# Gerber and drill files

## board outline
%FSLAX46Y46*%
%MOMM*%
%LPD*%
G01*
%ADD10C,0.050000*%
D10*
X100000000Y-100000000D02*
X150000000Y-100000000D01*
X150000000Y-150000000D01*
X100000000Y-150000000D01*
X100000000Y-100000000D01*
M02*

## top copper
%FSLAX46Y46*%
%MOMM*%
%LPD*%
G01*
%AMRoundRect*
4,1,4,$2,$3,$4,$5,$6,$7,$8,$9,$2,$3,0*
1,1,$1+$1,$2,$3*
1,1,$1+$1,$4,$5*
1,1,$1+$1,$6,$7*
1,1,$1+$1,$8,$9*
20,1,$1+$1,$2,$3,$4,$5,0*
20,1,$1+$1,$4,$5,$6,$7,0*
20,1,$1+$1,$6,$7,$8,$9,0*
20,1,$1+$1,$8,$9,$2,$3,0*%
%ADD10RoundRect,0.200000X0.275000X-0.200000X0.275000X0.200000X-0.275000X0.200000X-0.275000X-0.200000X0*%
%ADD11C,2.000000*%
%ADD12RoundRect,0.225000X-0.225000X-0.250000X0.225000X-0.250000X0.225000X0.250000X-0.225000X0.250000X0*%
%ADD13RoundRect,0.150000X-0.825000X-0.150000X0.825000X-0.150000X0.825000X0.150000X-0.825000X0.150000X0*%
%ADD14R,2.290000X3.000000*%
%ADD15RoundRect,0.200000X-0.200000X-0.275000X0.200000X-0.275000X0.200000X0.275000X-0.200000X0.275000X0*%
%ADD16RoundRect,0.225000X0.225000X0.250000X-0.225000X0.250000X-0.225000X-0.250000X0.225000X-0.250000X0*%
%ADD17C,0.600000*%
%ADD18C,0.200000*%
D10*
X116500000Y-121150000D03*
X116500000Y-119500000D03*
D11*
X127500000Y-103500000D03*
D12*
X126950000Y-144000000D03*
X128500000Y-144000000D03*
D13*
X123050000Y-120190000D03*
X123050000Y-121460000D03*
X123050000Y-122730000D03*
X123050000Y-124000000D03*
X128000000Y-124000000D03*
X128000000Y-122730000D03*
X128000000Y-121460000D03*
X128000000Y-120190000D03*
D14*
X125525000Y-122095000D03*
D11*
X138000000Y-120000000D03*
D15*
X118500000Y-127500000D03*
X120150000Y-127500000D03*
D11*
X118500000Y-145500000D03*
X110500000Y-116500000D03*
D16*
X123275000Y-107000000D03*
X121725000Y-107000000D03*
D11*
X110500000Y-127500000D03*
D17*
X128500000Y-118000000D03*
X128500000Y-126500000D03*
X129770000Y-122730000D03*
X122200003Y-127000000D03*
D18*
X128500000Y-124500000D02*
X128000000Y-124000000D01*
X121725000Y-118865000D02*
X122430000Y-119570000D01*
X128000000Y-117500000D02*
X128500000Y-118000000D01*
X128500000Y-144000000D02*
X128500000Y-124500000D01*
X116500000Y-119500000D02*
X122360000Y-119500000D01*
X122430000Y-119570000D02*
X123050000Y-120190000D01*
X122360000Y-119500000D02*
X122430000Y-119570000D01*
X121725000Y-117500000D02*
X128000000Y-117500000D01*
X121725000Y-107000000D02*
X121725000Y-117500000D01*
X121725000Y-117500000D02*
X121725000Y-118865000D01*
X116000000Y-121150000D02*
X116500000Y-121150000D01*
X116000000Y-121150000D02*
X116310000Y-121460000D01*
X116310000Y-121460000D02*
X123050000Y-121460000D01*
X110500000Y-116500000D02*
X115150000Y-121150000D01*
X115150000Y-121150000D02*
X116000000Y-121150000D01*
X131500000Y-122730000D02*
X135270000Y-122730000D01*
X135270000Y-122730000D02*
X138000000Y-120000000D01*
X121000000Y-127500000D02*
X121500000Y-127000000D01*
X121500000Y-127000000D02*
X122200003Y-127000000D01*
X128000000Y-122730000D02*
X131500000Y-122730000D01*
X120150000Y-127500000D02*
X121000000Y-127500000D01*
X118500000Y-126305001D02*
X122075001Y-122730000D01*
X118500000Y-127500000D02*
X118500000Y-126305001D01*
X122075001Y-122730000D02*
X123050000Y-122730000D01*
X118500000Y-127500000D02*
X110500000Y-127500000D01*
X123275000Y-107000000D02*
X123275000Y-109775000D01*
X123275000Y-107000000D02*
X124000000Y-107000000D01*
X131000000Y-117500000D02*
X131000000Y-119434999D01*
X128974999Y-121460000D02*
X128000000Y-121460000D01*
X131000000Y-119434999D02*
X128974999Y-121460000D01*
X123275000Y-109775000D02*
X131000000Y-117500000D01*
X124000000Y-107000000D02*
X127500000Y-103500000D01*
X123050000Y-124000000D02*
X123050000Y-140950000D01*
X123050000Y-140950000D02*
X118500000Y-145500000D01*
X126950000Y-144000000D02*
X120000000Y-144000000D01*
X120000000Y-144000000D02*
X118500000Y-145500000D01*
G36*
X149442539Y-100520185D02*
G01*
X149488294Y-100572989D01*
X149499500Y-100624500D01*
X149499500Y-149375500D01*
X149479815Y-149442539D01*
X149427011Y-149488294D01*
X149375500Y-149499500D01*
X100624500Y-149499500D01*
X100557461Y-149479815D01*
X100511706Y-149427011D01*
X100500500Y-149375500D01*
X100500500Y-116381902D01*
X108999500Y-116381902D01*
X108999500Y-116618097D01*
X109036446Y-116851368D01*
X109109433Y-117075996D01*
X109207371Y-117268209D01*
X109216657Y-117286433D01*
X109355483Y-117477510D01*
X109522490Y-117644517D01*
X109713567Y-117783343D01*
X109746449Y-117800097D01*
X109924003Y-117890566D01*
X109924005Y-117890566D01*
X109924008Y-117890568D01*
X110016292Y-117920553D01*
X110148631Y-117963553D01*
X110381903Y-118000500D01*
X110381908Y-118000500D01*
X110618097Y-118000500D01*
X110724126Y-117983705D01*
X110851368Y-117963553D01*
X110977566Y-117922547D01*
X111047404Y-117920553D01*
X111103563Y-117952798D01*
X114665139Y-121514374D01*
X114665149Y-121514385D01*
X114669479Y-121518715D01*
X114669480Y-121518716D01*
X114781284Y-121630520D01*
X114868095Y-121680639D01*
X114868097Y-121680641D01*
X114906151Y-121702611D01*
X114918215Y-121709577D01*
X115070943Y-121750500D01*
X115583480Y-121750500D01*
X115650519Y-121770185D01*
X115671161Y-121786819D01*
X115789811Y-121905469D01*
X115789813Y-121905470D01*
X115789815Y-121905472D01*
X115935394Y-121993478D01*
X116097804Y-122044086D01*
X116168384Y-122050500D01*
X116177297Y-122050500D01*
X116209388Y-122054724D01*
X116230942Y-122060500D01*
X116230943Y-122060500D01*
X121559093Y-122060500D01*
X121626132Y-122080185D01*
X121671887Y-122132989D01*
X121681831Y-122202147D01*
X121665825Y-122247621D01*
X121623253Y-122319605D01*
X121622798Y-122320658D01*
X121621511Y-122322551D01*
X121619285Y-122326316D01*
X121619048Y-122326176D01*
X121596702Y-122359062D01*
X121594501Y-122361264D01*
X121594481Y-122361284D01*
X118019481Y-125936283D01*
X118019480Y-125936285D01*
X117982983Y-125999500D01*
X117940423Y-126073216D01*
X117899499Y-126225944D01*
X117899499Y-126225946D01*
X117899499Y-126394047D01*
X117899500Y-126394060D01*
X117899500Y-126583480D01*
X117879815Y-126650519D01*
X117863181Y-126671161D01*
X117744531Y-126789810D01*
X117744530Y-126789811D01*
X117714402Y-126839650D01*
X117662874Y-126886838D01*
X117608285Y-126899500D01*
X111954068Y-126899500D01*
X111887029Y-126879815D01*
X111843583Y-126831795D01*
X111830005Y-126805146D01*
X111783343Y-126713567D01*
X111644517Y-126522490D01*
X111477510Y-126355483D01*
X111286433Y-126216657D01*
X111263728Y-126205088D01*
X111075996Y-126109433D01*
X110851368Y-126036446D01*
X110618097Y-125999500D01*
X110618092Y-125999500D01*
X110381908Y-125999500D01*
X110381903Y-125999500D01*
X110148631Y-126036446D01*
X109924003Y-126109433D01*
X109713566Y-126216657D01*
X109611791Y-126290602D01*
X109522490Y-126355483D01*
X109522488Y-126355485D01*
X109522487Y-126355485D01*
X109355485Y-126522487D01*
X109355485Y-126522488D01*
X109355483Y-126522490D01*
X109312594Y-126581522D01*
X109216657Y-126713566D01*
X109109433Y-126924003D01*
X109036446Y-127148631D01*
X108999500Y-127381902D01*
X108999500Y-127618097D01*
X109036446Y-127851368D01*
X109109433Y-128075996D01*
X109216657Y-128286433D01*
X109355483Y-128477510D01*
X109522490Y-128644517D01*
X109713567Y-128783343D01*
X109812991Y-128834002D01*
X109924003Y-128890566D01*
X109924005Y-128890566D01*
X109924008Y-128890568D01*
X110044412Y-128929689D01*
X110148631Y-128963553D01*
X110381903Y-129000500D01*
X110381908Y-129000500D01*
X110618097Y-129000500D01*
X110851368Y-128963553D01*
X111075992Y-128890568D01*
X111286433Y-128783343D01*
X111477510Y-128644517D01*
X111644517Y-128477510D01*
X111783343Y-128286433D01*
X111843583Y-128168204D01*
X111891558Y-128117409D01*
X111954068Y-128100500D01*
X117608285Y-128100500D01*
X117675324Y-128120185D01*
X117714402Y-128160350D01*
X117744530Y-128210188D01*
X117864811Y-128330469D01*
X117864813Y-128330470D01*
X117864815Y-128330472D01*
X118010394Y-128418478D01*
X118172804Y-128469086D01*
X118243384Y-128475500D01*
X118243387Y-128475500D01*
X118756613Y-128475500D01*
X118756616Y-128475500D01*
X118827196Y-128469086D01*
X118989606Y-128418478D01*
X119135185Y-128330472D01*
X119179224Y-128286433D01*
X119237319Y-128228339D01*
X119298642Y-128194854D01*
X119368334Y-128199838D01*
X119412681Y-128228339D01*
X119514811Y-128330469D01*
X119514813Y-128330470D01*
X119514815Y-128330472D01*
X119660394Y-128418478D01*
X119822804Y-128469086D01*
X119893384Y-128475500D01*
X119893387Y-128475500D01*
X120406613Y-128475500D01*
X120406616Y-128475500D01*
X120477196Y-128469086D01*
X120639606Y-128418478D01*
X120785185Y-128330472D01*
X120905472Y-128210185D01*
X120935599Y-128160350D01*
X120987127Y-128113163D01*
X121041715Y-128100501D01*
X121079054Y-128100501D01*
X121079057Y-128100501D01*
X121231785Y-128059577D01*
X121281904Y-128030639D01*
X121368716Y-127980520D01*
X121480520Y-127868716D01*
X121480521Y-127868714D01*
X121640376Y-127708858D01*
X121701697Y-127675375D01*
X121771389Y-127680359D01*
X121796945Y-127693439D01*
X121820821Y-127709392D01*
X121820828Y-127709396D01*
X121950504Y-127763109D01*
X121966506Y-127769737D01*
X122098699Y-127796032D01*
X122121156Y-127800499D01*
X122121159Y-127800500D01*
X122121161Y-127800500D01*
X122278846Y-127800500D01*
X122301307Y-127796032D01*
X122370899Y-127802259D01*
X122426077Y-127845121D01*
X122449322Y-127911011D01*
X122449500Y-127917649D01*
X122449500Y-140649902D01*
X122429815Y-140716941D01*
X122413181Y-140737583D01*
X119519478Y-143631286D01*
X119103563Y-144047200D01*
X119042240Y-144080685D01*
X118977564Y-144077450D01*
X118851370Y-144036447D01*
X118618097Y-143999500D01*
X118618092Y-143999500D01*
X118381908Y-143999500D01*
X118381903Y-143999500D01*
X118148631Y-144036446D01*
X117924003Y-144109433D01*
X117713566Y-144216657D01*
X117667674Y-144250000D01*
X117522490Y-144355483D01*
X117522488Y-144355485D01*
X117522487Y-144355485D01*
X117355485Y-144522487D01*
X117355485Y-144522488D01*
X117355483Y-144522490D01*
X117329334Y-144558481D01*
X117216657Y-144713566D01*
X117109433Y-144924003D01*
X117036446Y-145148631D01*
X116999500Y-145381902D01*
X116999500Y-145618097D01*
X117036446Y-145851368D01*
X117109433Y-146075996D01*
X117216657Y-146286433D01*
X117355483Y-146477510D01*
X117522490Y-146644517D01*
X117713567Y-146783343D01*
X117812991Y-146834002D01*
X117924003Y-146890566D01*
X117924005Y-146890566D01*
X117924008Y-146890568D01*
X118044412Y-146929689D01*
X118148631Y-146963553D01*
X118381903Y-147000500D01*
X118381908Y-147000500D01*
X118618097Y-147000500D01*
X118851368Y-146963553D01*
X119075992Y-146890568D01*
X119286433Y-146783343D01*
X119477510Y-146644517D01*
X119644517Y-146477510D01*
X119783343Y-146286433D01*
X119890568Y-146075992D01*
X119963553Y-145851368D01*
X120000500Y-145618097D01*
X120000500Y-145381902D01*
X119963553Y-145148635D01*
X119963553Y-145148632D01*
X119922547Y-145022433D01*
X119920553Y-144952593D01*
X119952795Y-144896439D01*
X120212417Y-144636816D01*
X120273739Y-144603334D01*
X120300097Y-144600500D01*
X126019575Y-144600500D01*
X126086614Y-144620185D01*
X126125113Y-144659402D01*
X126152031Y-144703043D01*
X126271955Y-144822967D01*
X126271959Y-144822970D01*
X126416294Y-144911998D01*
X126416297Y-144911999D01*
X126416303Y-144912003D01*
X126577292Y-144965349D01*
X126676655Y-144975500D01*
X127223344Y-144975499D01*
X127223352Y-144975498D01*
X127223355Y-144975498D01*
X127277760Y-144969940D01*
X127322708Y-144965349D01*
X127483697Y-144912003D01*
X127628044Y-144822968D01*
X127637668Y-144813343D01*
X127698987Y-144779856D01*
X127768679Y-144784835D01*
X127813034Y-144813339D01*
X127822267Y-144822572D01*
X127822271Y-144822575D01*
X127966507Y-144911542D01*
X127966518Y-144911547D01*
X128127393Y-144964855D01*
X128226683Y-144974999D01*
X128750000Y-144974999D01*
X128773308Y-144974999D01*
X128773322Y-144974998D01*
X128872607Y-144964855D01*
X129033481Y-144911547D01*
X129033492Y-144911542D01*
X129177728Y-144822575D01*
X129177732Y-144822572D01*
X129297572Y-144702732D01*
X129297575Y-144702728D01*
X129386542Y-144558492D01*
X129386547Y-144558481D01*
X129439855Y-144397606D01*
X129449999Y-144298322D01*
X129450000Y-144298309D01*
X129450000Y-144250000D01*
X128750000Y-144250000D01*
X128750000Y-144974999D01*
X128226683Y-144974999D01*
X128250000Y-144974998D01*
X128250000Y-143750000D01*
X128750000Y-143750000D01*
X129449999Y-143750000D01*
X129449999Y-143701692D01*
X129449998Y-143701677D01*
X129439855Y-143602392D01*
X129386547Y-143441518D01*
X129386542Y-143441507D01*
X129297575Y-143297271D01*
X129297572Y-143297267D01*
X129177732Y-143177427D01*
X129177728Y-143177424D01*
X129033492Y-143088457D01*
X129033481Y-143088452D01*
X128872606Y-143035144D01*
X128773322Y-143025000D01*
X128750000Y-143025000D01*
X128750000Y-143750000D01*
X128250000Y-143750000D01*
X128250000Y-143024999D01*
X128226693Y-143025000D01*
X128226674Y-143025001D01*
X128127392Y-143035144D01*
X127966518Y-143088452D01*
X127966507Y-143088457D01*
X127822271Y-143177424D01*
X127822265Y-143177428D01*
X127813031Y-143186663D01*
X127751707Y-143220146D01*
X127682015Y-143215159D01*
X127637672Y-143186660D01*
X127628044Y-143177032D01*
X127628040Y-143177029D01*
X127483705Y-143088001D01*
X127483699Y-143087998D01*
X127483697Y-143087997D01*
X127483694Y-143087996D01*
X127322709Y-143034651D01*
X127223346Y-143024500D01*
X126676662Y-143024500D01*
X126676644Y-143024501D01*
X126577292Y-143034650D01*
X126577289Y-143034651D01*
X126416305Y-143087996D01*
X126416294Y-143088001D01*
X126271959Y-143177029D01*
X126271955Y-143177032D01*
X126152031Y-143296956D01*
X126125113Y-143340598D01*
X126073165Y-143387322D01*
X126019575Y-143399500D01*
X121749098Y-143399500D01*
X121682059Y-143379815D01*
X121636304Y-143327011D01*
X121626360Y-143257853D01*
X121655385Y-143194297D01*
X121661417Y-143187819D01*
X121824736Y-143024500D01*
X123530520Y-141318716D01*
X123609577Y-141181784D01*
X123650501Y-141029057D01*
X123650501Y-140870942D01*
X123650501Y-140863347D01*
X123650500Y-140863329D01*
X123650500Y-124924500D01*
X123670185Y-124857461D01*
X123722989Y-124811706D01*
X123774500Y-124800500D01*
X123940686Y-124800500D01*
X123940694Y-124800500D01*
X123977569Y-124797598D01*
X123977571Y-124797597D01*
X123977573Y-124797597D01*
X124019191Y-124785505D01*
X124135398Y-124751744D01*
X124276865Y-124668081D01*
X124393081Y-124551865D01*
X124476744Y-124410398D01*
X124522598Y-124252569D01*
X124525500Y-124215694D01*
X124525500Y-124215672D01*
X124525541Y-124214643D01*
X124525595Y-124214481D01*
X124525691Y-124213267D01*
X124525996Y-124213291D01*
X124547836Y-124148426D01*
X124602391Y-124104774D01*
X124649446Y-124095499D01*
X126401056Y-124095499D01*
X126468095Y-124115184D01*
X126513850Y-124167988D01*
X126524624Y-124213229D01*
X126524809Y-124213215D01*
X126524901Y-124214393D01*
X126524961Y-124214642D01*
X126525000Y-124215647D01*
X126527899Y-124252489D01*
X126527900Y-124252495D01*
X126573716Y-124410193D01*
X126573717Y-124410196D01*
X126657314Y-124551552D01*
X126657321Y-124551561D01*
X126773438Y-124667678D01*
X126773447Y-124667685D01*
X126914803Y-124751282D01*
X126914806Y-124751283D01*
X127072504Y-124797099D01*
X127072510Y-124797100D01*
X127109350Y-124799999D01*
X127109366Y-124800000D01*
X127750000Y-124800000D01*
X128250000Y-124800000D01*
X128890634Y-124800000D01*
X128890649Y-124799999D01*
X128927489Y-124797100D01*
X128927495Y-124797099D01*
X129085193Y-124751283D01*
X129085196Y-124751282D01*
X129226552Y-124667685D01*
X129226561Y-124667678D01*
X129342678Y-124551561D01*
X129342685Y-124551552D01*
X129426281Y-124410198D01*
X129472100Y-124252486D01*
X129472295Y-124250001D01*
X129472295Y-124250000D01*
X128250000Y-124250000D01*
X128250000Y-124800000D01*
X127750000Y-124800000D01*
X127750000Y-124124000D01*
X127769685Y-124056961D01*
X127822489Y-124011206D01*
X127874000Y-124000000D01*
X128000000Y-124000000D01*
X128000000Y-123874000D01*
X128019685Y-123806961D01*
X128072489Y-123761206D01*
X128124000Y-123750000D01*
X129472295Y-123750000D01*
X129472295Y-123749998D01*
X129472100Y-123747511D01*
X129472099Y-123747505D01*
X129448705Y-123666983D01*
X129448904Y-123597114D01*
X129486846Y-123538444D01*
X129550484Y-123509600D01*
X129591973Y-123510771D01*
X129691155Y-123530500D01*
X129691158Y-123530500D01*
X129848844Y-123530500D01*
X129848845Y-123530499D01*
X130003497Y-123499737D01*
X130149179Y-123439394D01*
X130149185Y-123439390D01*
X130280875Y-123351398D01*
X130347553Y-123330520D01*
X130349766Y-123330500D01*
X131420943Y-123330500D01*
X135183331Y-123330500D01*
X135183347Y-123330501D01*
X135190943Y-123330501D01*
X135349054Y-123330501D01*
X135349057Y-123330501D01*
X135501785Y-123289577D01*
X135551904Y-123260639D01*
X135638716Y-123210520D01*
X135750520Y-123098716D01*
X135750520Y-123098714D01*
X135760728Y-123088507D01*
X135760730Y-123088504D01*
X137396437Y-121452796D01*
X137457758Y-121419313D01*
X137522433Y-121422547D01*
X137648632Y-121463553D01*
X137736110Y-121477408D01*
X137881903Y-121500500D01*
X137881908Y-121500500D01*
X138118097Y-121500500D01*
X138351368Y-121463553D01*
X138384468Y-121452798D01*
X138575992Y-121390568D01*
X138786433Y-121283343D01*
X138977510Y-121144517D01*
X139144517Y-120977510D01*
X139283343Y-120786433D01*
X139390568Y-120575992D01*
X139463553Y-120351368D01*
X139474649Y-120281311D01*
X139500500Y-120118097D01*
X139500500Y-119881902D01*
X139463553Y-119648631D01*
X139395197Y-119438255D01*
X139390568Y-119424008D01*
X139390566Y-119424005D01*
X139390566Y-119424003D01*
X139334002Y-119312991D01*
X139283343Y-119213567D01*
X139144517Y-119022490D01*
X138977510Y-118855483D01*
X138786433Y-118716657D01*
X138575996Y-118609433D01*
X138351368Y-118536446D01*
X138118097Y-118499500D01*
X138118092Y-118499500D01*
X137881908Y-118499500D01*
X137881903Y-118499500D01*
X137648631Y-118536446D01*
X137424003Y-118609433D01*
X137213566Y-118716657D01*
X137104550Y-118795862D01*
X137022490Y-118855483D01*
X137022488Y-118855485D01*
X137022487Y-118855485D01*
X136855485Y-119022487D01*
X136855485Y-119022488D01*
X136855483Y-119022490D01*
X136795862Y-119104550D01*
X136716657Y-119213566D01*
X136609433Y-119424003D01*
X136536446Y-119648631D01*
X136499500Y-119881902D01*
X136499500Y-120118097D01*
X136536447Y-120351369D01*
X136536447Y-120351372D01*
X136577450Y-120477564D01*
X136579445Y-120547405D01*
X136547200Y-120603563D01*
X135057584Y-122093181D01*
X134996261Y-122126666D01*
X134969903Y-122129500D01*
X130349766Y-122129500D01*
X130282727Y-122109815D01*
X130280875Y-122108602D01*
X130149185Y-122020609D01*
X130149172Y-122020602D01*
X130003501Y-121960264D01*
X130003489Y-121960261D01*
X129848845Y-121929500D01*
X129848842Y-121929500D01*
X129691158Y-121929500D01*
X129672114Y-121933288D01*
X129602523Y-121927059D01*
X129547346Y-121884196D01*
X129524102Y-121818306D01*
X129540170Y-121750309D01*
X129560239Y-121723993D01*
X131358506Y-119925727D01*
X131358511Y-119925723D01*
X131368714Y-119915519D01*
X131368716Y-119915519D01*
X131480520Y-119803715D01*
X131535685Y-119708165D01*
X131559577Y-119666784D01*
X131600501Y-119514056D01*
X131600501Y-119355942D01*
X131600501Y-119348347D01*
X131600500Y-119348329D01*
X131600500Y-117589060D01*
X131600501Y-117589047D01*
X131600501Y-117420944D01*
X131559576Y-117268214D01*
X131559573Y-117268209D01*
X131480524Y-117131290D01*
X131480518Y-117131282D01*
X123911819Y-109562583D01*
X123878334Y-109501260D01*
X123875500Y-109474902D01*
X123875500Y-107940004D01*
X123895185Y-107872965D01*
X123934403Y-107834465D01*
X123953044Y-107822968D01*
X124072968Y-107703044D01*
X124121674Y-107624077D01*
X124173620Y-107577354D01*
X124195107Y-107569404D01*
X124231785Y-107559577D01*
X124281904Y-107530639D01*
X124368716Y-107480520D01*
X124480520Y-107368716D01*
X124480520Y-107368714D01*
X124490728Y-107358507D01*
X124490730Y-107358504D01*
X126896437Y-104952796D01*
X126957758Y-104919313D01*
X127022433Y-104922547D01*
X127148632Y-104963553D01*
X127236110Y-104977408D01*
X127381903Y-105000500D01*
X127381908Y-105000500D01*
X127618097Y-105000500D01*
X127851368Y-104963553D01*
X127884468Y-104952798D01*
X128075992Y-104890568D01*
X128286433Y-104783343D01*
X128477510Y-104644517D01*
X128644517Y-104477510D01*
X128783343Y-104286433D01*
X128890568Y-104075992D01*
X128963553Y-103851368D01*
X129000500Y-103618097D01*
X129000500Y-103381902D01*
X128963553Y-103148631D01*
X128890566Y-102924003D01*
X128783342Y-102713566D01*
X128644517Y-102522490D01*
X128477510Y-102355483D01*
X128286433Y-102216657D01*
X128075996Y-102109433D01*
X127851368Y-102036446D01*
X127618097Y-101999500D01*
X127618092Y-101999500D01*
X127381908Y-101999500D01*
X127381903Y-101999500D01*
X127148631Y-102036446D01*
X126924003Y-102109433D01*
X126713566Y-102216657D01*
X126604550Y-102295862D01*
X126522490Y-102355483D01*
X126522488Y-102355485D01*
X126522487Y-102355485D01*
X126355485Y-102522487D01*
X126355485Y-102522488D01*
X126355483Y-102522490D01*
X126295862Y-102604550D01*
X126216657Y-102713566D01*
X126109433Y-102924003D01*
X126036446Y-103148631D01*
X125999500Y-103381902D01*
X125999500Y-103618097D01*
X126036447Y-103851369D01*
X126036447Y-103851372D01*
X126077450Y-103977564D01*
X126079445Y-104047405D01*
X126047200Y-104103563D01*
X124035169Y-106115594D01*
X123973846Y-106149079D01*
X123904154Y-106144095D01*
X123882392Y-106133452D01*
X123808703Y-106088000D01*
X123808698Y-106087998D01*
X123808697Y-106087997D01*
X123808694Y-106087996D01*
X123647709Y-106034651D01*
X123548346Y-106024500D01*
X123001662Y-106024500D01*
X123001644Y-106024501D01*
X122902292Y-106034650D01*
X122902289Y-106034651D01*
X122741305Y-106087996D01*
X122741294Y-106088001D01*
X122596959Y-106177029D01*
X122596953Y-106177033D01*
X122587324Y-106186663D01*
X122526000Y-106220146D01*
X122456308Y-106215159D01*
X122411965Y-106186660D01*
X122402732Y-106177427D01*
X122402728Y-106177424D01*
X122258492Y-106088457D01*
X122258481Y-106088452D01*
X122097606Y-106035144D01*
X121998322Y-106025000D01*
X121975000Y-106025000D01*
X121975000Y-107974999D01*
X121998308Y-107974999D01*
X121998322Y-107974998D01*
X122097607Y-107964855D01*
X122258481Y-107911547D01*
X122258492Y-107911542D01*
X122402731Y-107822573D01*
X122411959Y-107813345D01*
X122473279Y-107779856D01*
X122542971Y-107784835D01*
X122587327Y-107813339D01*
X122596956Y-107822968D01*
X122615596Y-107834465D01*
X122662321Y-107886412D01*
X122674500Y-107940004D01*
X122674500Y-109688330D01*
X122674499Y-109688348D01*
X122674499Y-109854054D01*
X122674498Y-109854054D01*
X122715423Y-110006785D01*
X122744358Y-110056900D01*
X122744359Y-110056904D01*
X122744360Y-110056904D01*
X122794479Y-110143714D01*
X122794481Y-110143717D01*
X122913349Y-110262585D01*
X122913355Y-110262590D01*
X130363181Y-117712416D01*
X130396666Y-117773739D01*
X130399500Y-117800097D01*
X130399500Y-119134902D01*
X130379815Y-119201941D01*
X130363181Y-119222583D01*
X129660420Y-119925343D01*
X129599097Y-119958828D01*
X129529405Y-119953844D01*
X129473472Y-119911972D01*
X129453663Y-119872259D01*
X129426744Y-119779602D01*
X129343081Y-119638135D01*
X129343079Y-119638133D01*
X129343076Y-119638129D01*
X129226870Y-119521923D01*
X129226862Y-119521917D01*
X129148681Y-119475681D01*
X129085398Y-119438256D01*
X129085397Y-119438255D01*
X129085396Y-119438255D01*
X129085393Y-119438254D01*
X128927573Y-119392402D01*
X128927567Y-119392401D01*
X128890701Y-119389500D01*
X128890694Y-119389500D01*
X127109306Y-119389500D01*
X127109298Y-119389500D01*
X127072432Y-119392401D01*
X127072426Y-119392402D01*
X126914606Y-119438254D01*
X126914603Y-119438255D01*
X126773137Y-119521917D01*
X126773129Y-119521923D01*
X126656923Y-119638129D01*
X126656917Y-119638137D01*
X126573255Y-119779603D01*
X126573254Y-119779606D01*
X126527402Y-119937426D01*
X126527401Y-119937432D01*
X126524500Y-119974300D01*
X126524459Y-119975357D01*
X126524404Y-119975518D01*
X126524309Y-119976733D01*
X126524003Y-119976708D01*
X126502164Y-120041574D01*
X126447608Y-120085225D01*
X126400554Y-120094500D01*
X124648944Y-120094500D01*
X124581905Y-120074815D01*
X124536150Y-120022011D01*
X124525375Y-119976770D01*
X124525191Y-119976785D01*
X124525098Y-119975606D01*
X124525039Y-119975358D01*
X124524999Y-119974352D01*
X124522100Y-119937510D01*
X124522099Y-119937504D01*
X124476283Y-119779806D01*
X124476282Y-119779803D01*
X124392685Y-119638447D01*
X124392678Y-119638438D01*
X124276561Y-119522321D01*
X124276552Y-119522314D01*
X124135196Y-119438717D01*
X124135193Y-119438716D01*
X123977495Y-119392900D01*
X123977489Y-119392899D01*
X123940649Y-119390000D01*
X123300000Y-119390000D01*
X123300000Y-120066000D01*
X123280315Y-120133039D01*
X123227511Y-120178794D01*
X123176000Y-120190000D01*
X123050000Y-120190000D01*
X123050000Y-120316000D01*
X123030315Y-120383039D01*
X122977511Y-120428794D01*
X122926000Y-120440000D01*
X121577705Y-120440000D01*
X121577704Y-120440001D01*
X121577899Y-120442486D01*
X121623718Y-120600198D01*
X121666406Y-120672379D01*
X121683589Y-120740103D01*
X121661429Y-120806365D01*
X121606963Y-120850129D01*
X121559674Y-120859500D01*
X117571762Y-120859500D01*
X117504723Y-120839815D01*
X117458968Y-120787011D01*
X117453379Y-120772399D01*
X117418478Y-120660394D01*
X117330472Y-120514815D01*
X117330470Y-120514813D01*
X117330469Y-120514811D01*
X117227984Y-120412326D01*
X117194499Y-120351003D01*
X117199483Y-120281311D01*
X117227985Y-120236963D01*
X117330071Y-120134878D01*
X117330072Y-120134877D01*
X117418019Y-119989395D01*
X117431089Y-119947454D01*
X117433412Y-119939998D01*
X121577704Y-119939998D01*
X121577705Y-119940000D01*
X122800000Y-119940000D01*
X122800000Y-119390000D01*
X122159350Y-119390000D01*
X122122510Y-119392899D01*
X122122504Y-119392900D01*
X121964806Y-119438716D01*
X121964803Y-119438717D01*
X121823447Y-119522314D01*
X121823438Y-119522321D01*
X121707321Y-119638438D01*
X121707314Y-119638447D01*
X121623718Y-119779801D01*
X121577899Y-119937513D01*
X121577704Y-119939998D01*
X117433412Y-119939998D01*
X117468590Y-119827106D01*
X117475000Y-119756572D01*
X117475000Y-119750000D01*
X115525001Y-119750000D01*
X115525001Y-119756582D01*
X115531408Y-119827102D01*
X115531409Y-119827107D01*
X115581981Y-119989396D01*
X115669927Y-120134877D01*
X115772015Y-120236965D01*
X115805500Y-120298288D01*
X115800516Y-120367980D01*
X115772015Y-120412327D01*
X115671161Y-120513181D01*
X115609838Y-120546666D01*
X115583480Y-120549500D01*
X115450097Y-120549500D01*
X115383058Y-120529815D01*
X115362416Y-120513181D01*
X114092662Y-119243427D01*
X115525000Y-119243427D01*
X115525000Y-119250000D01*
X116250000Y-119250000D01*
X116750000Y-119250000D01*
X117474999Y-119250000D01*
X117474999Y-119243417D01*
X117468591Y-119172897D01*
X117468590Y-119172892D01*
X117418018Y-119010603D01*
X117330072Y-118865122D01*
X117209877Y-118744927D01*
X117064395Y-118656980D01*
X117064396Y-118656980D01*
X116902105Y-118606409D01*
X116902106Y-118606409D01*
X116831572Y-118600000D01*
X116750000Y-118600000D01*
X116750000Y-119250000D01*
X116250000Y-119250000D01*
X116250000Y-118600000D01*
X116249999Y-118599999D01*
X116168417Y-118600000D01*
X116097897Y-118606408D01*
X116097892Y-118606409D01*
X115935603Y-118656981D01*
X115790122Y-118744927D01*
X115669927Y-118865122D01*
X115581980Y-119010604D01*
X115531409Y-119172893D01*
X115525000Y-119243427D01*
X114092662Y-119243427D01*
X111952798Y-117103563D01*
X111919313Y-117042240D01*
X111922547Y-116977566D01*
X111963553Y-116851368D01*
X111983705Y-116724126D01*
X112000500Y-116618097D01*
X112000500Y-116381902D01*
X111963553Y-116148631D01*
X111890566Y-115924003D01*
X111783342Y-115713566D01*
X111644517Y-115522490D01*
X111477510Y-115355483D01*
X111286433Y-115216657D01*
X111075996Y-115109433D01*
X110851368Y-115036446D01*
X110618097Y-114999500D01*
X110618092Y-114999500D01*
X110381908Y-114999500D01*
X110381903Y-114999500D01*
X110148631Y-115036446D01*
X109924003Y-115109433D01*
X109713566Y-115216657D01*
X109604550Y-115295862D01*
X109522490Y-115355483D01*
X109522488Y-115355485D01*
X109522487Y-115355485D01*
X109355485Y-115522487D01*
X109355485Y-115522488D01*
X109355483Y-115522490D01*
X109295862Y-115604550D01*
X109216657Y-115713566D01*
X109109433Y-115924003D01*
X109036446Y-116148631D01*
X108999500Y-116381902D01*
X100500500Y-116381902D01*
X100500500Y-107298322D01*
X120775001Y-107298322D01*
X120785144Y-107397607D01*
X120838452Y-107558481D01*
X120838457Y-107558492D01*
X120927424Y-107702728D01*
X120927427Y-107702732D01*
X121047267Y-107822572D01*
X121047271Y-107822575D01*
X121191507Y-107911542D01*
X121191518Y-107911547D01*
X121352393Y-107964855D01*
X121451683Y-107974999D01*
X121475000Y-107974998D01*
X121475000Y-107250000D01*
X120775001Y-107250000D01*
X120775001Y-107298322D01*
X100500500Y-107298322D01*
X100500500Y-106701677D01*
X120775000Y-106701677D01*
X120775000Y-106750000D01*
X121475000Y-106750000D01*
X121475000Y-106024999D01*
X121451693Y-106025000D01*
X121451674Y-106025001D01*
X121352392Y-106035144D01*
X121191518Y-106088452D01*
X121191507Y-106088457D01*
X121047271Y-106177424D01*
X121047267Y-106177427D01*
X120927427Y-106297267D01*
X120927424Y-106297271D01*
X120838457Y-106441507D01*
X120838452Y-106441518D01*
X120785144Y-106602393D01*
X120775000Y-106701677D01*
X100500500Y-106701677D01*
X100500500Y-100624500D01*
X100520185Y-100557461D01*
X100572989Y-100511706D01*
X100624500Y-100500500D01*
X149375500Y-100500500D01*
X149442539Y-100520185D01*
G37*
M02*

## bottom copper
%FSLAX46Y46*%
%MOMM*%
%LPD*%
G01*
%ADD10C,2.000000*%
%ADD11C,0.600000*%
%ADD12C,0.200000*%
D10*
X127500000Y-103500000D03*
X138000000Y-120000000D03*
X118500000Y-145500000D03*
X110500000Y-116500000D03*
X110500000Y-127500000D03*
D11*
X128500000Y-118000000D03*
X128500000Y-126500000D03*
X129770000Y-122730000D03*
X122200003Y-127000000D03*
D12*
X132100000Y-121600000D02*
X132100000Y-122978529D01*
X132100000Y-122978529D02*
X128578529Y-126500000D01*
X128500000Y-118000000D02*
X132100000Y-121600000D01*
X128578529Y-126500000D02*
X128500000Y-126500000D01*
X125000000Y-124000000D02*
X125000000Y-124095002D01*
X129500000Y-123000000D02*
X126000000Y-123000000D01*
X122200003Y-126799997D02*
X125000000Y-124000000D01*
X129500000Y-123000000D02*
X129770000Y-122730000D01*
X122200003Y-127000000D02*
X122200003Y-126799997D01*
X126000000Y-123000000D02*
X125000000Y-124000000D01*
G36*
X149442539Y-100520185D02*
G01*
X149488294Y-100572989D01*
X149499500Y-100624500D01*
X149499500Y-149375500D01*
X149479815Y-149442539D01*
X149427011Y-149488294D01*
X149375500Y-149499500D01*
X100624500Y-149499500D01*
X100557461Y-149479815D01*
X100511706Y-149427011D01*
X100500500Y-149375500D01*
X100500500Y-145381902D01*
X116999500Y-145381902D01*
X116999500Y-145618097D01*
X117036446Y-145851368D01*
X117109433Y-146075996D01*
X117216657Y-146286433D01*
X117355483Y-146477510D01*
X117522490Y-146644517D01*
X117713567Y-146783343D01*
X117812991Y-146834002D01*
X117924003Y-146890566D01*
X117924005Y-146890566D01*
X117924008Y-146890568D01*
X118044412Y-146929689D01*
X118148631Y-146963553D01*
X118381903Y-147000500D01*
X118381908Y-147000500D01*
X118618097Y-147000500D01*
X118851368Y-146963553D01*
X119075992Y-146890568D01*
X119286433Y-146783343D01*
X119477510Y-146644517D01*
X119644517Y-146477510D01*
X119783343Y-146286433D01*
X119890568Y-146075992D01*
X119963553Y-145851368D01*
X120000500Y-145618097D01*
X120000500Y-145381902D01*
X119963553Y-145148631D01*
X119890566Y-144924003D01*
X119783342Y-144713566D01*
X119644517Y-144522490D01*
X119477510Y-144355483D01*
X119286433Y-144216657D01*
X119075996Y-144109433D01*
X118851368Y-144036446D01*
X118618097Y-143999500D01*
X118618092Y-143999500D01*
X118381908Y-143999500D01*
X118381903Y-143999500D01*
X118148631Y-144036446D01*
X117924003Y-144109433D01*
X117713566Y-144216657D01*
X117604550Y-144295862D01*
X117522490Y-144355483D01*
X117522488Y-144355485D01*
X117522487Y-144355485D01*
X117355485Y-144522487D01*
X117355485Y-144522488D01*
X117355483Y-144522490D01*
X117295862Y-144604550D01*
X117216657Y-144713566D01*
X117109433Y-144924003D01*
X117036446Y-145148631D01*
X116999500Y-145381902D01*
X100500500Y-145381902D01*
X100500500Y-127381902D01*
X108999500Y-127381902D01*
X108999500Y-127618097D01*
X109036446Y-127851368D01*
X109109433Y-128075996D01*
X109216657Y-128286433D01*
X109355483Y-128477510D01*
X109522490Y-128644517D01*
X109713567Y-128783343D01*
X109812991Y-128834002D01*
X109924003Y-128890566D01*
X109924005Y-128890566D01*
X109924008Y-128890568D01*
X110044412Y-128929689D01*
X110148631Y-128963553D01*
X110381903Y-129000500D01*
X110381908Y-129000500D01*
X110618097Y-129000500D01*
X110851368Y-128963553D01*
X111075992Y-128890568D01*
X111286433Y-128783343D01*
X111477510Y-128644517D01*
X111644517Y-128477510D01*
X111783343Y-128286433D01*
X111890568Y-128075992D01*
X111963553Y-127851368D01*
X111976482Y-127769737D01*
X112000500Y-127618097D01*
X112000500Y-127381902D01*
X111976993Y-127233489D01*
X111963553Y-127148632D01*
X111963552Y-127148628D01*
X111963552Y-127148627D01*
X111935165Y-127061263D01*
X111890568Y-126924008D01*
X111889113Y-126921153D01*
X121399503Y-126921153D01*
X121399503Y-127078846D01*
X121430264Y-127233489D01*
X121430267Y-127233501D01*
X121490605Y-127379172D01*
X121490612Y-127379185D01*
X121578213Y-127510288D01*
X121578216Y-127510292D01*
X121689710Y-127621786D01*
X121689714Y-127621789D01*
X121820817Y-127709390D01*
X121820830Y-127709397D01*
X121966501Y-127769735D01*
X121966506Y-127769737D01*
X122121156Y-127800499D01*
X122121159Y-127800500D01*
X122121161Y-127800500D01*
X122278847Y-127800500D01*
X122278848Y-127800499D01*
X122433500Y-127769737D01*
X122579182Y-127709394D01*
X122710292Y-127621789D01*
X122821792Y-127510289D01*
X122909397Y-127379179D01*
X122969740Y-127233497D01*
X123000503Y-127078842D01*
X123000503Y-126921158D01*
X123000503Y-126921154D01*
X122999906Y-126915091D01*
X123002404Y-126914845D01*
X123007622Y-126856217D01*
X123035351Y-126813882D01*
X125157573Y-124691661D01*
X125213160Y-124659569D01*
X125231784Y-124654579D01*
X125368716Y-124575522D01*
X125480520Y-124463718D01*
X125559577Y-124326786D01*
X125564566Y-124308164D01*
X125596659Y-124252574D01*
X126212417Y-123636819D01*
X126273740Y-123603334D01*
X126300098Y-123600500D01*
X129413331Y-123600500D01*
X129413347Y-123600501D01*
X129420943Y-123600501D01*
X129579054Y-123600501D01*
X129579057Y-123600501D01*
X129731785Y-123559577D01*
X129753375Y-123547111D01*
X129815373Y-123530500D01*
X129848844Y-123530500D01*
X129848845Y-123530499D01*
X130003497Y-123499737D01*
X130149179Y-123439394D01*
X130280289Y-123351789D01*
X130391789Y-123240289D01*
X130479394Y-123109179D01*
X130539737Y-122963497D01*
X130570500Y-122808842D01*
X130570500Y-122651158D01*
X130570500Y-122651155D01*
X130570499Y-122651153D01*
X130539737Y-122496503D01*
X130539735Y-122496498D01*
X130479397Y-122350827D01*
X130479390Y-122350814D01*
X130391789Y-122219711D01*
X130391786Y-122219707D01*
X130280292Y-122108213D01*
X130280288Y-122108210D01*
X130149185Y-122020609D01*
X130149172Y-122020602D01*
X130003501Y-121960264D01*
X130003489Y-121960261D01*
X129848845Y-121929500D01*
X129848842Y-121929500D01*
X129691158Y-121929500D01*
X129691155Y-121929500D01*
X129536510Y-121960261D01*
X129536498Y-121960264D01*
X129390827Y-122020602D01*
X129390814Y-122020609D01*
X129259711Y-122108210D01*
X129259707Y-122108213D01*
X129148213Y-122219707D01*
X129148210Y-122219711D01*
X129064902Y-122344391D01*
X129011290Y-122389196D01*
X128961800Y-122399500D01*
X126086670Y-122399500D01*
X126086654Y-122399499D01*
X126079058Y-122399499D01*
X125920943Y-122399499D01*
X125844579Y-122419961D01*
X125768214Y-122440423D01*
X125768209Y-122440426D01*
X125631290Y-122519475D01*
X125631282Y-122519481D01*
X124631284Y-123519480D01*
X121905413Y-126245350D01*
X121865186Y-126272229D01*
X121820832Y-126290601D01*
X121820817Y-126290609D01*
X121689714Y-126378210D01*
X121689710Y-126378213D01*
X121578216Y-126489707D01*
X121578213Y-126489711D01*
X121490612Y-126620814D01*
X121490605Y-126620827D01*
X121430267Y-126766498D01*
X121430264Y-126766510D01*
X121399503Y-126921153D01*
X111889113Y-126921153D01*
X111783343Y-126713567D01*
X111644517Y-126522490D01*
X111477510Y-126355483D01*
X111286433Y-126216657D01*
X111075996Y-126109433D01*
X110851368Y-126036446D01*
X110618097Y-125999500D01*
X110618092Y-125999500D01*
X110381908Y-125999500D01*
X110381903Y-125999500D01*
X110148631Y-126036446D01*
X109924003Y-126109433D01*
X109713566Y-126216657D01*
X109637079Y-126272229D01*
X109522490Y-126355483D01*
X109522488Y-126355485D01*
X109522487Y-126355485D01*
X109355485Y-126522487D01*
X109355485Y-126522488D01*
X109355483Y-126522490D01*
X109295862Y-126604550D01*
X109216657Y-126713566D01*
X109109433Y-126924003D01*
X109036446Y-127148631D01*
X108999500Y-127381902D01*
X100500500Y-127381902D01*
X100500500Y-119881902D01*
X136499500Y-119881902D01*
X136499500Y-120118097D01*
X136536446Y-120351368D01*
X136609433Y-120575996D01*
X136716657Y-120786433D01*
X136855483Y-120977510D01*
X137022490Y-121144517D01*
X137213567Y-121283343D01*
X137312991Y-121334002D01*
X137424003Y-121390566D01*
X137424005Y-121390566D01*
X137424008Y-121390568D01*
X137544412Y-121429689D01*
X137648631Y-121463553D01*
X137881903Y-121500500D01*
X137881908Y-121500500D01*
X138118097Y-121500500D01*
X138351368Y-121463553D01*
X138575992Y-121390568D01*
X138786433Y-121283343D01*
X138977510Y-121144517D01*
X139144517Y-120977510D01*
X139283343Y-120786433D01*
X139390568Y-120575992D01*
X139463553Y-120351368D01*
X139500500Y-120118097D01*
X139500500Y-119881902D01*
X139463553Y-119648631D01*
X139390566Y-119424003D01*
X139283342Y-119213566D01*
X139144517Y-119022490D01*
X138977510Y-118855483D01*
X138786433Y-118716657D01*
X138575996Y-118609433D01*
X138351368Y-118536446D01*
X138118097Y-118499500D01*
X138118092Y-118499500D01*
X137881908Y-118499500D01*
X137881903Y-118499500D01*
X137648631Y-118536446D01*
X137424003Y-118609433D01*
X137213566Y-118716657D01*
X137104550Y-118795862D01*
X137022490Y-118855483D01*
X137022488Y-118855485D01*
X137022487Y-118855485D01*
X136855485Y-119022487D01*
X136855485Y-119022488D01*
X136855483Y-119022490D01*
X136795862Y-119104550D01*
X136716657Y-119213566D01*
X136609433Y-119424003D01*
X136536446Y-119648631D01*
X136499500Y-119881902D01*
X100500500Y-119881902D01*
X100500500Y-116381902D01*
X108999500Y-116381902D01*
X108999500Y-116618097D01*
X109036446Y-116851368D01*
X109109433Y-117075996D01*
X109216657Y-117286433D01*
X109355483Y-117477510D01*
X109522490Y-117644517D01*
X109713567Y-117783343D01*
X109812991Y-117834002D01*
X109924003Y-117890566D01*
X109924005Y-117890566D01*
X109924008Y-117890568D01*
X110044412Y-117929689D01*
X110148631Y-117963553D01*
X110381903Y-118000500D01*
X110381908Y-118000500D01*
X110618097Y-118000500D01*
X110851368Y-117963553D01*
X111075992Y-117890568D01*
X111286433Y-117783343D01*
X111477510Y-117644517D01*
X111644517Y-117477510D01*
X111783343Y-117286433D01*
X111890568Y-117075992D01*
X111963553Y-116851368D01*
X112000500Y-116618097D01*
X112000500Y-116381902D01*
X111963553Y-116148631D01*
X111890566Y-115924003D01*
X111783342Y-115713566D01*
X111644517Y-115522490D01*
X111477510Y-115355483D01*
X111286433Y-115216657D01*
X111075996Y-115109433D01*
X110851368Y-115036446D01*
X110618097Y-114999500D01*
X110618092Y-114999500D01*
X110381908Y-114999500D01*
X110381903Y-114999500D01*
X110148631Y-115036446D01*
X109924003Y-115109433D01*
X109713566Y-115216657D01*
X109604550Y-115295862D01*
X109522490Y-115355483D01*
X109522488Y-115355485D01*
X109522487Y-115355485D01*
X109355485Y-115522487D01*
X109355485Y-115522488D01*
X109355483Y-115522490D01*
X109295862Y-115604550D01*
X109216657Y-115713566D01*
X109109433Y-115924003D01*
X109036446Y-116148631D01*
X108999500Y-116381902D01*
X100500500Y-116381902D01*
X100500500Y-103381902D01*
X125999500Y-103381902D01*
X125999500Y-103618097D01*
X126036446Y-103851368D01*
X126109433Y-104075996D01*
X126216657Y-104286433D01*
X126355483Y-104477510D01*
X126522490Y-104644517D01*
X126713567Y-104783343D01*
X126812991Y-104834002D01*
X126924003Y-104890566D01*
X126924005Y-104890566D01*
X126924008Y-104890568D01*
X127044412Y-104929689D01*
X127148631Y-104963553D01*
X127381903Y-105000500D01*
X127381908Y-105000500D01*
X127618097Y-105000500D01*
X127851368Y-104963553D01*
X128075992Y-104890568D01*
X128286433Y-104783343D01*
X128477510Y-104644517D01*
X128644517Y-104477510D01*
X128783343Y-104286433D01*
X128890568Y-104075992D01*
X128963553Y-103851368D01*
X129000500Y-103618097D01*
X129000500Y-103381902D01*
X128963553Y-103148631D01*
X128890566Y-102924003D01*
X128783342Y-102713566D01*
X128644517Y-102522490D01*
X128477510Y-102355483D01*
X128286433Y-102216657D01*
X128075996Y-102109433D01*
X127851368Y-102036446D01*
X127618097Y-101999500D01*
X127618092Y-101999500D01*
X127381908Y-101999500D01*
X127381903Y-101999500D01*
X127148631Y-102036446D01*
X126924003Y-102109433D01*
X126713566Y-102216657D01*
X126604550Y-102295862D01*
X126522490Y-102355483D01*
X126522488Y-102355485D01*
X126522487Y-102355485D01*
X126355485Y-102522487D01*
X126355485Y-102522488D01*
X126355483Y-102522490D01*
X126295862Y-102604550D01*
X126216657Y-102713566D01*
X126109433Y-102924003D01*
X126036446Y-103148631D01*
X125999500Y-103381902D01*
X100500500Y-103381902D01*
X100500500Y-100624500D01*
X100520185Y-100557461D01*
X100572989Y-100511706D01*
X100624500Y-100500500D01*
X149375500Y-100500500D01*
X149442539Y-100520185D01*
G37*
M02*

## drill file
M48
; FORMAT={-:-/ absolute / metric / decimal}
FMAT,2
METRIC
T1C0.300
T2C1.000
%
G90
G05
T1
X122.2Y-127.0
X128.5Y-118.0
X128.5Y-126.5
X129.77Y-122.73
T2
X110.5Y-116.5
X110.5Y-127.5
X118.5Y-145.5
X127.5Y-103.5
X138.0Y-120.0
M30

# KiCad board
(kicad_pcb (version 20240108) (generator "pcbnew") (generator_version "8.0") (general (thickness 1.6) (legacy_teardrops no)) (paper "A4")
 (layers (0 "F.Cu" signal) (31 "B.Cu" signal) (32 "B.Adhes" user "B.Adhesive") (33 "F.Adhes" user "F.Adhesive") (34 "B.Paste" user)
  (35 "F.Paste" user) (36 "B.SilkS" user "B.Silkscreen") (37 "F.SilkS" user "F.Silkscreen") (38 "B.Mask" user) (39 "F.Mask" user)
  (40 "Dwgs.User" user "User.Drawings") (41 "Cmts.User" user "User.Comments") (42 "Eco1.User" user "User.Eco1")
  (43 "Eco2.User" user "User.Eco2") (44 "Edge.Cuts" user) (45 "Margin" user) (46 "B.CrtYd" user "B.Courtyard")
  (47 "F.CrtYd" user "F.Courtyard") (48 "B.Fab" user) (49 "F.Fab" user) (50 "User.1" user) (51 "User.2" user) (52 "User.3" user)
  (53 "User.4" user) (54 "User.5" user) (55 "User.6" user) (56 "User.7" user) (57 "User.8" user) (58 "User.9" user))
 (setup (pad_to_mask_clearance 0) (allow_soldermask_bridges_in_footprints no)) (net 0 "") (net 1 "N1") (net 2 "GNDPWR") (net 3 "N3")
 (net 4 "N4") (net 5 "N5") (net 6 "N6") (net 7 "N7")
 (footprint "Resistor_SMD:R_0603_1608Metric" (layer "F.Cu") (at 116.5 120.325 90)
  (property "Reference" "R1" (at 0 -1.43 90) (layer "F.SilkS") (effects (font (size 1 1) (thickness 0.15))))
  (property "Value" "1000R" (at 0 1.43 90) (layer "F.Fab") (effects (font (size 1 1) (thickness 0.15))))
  (pad "1" smd roundrect (at -0.825 0 90) (size 0.8 0.95) (layers "F.Cu" "F.Paste" "F.Mask") (roundrect_rratio 0.25) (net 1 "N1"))
  (pad "2" smd roundrect (at 0.825 0 90) (size 0.8 0.95) (layers "F.Cu" "F.Paste" "F.Mask") (roundrect_rratio 0.25) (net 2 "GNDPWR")))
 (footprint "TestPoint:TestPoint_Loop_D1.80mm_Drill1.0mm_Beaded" (layer "F.Cu") (at 127.5 103.5)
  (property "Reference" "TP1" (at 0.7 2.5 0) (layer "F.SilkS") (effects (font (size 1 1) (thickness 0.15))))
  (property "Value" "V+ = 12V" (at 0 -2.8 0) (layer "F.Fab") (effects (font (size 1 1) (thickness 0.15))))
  (pad "1" thru_hole circle (at 0 0) (size 2 2) (drill 1) (layers "*.Cu" "*.Mask") (remove_unused_layers no) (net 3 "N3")))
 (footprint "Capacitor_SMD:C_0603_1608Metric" (layer "F.Cu") (at 127.725 144)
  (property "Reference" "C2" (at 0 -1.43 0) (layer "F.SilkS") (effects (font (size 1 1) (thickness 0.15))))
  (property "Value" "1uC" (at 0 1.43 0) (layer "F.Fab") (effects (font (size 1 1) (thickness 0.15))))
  (pad "1" smd roundrect (at -0.775 0) (size 0.9 0.95) (layers "F.Cu" "F.Paste" "F.Mask") (roundrect_rratio 0.25) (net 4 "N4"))
  (pad "2" smd roundrect (at 0.775 0) (size 0.9 0.95) (layers "F.Cu" "F.Paste" "F.Mask") (roundrect_rratio 0.25) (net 2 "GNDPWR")))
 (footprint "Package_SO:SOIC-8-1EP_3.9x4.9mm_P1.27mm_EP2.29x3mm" (layer "F.Cu") (at 125.525 122.095)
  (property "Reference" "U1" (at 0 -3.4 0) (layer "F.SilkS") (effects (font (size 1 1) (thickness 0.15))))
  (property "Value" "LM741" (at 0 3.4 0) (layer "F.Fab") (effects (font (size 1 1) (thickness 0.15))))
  (pad "" smd roundrect (at -0.57 -0.75) (size 0.92 1.21) (layers "F.Paste") (roundrect_rratio 0.25))
  (pad "" smd roundrect (at -0.57 0.75) (size 0.92 1.21) (layers "F.Paste") (roundrect_rratio 0.25))
  (pad "" smd roundrect (at 0.57 -0.75) (size 0.92 1.21) (layers "F.Paste") (roundrect_rratio 0.25))
  (pad "" smd roundrect (at 0.57 0.75) (size 0.92 1.21) (layers "F.Paste") (roundrect_rratio 0.25))
  (pad "1" smd roundrect (at -2.475 -1.905) (size 1.95 0.6) (layers "F.Cu" "F.Paste" "F.Mask") (roundrect_rratio 0.25) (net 2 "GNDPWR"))
  (pad "2" smd roundrect (at -2.475 -0.635) (size 1.95 0.6) (layers "F.Cu" "F.Paste" "F.Mask") (roundrect_rratio 0.25) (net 1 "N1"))
  (pad "3" smd roundrect (at -2.475 0.635) (size 1.95 0.6) (layers "F.Cu" "F.Paste" "F.Mask") (roundrect_rratio 0.25) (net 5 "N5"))
  (pad "4" smd roundrect (at -2.475 1.905) (size 1.95 0.6) (layers "F.Cu" "F.Paste" "F.Mask") (roundrect_rratio 0.25) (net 4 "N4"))
  (pad "5" smd roundrect (at 2.475 1.905) (size 1.95 0.6) (layers "F.Cu" "F.Paste" "F.Mask") (roundrect_rratio 0.25) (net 2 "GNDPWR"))
  (pad "6" smd roundrect (at 2.475 0.635) (size 1.95 0.6) (layers "F.Cu" "F.Paste" "F.Mask") (roundrect_rratio 0.25) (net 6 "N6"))
  (pad "7" smd roundrect (at 2.475 -0.635) (size 1.95 0.6) (layers "F.Cu" "F.Paste" "F.Mask") (roundrect_rratio 0.25) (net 3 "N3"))
  (pad "8" smd roundrect (at 2.475 -1.905) (size 1.95 0.6) (layers "F.Cu" "F.Paste" "F.Mask") (roundrect_rratio 0.25) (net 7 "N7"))
  (pad "9" smd rect (at 0 0) (size 2.29 3) (layers "F.Cu" "F.Mask") (zone_connect 2)))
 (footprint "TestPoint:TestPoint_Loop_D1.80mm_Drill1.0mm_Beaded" (layer "F.Cu") (at 138 120)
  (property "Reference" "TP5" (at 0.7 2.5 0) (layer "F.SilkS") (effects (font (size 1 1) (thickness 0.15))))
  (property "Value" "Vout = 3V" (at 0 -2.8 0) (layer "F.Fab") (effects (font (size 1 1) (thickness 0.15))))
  (pad "1" thru_hole circle (at 0 0) (size 2 2) (drill 1) (layers "*.Cu" "*.Mask") (remove_unused_layers no) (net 6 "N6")))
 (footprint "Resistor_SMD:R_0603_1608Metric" (layer "F.Cu") (at 119.325 127.5)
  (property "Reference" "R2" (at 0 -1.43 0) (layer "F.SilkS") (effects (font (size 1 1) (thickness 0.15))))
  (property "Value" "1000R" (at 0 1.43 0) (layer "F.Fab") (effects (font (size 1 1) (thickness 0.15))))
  (pad "1" smd roundrect (at -0.825 0) (size 0.8 0.95) (layers "F.Cu" "F.Paste" "F.Mask") (roundrect_rratio 0.25) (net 5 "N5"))
  (pad "2" smd roundrect (at 0.825 0) (size 0.8 0.95) (layers "F.Cu" "F.Paste" "F.Mask") (roundrect_rratio 0.25) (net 6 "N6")))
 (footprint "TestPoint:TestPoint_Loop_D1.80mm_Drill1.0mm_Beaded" (layer "F.Cu") (at 118.5 145.5)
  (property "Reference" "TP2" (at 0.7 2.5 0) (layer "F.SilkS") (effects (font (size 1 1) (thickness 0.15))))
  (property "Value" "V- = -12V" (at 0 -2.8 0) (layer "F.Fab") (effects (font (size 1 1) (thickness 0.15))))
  (pad "1" thru_hole circle (at 0 0) (size 2 2) (drill 1) (layers "*.Cu" "*.Mask") (remove_unused_layers no) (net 4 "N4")))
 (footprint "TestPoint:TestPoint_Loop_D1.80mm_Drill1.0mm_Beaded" (layer "F.Cu") (at 110.5 116.5)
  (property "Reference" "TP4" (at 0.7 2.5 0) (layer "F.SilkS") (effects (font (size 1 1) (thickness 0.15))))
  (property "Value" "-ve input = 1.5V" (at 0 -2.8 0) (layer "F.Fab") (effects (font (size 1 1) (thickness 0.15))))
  (pad "1" thru_hole circle (at 0 0) (size 2 2) (drill 1) (layers "*.Cu" "*.Mask") (remove_unused_layers no) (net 1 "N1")))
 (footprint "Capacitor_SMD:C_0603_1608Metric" (layer "F.Cu") (at 122.5 107 180)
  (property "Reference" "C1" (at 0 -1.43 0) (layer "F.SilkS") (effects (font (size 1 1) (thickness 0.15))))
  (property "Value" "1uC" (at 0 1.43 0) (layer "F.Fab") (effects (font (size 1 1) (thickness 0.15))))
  (pad "1" smd roundrect (at -0.775 0 180) (size 0.9 0.95) (layers "F.Cu" "F.Paste" "F.Mask") (roundrect_rratio 0.25) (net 3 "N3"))
  (pad "2" smd roundrect (at 0.775 0 180) (size 0.9 0.95) (layers "F.Cu" "F.Paste" "F.Mask") (roundrect_rratio 0.25) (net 2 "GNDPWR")))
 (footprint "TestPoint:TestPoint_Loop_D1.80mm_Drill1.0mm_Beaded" (layer "F.Cu") (at 110.5 127.5)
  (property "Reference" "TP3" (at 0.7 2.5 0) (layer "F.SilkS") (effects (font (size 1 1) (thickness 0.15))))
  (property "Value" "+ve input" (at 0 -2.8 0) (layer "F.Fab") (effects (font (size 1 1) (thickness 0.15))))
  (pad "1" thru_hole circle (at 0 0) (size 2 2) (drill 1) (layers "*.Cu" "*.Mask") (remove_unused_layers no) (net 5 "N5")))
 (gr_rect (start 100 100) (end 150 150) (stroke (width 0.05) (type default)) (fill none) (layer "Edge.Cuts"))
 (segment (start 128.5 124.5) (end 128 124) (width 0.2) (layer "F.Cu") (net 2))
 (segment (start 121.725 118.865) (end 122.43 119.57) (width 0.2) (layer "F.Cu") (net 2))
 (segment (start 128 117.5) (end 128.5 118) (width 0.2) (layer "F.Cu") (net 2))
 (segment (start 128.5 144) (end 128.5 124.5) (width 0.2) (layer "F.Cu") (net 2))
 (segment (start 116.5 119.5) (end 122.36 119.5) (width 0.2) (layer "F.Cu") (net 2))
 (segment (start 122.43 119.57) (end 123.05 120.19) (width 0.2) (layer "F.Cu") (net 2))
 (segment (start 122.36 119.5) (end 122.43 119.57) (width 0.2) (layer "F.Cu") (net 2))
 (segment (start 121.725 117.5) (end 128 117.5) (width 0.2) (layer "F.Cu") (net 2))
 (segment (start 121.725 107) (end 121.725 117.5) (width 0.2) (layer "F.Cu") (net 2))
 (segment (start 121.725 117.5) (end 121.725 118.865) (width 0.2) (layer "F.Cu") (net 2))
 (via (at 128.5 118) (size 0.6) (drill 0.3) (layers "F.Cu" "B.Cu") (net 2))
 (via (at 128.5 126.5) (size 0.6) (drill 0.3) (layers "F.Cu" "B.Cu") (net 2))
 (segment (start 132.1 121.6) (end 132.1 122.978529) (width 0.2) (layer "B.Cu") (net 2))
 (segment (start 132.1 122.978529) (end 128.578529 126.5) (width 0.2) (layer "B.Cu") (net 2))
 (segment (start 128.5 118) (end 132.1 121.6) (width 0.2) (layer "B.Cu") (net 2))
 (segment (start 128.578529 126.5) (end 128.5 126.5) (width 0.2) (layer "B.Cu") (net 2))
 (segment (start 116 121.15) (end 116.5 121.15) (width 0.2) (layer "F.Cu") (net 1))
 (segment (start 116 121.15) (end 116.31 121.46) (width 0.2) (layer "F.Cu") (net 1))
 (segment (start 116.31 121.46) (end 123.05 121.46) (width 0.2) (layer "F.Cu") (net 1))
 (segment (start 110.5 116.5) (end 115.15 121.15) (width 0.2) (layer "F.Cu") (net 1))
 (segment (start 115.15 121.15) (end 116 121.15) (width 0.2) (layer "F.Cu") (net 1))
 (segment (start 131.5 122.73) (end 135.27 122.73) (width 0.2) (layer "F.Cu") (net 6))
 (segment (start 135.27 122.73) (end 138 120) (width 0.2) (layer "F.Cu") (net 6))
 (segment (start 121 127.5) (end 121.5 127) (width 0.2) (layer "F.Cu") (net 6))
 (segment (start 121.5 127) (end 122.200003 127) (width 0.2) (layer "F.Cu") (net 6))
 (segment (start 128 122.73) (end 131.5 122.73) (width 0.2) (layer "F.Cu") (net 6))
 (segment (start 120.15 127.5) (end 121 127.5) (width 0.2) (layer "F.Cu") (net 6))
 (via (at 129.77 122.73) (size 0.6) (drill 0.3) (layers "F.Cu" "B.Cu") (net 6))
 (via (at 122.200003 127) (size 0.6) (drill 0.3) (layers "F.Cu" "B.Cu") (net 6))
 (segment (start 125 124) (end 125 124.095002) (width 0.2) (layer "B.Cu") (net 6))
 (segment (start 129.5 123) (end 126 123) (width 0.2) (layer "B.Cu") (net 6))
 (segment (start 122.200003 126.799997) (end 125 124) (width 0.2) (layer "B.Cu") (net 6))
 (segment (start 129.5 123) (end 129.77 122.73) (width 0.2) (layer "B.Cu") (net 6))
 (segment (start 122.200003 127) (end 122.200003 126.799997) (width 0.2) (layer "B.Cu") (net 6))
 (segment (start 126 123) (end 125 124) (width 0.2) (layer "B.Cu") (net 6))
 (segment (start 118.5 126.305001) (end 122.075001 122.73) (width 0.2) (layer "F.Cu") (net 5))
 (segment (start 118.5 127.5) (end 118.5 126.305001) (width 0.2) (layer "F.Cu") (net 5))
 (segment (start 122.075001 122.73) (end 123.05 122.73) (width 0.2) (layer "F.Cu") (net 5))
 (segment (start 118.5 127.5) (end 110.5 127.5) (width 0.2) (layer "F.Cu") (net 5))
 (segment (start 123.275 107) (end 123.275 109.775) (width 0.2) (layer "F.Cu") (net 3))
 (segment (start 123.275 107) (end 124 107) (width 0.2) (layer "F.Cu") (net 3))
 (segment (start 131 117.5) (end 131 119.434999) (width 0.2) (layer "F.Cu") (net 3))
 (segment (start 128.974999 121.46) (end 128 121.46) (width 0.2) (layer "F.Cu") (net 3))
 (segment (start 131 119.434999) (end 128.974999 121.46) (width 0.2) (layer "F.Cu") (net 3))
 (segment (start 123.275 109.775) (end 131 117.5) (width 0.2) (layer "F.Cu") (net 3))
 (segment (start 124 107) (end 127.5 103.5) (width 0.2) (layer "F.Cu") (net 3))
 (segment (start 123.05 124) (end 123.05 140.95) (width 0.2) (layer "F.Cu") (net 4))
 (segment (start 123.05 140.95) (end 118.5 145.5) (width 0.2) (layer "F.Cu") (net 4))
 (segment (start 126.95 144) (end 120 144) (width 0.2) (layer "F.Cu") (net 4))
 (segment (start 120 144) (end 118.5 145.5) (width 0.2) (layer "F.Cu") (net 4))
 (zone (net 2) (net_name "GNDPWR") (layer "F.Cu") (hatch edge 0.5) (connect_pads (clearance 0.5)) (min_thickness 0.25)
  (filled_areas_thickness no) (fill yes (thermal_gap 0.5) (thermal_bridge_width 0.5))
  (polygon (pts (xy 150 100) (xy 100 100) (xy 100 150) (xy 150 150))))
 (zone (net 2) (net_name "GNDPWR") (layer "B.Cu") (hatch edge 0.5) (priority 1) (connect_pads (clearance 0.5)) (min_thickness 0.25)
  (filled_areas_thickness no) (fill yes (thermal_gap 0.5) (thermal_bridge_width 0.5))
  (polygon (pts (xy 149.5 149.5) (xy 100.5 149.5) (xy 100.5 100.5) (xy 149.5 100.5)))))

